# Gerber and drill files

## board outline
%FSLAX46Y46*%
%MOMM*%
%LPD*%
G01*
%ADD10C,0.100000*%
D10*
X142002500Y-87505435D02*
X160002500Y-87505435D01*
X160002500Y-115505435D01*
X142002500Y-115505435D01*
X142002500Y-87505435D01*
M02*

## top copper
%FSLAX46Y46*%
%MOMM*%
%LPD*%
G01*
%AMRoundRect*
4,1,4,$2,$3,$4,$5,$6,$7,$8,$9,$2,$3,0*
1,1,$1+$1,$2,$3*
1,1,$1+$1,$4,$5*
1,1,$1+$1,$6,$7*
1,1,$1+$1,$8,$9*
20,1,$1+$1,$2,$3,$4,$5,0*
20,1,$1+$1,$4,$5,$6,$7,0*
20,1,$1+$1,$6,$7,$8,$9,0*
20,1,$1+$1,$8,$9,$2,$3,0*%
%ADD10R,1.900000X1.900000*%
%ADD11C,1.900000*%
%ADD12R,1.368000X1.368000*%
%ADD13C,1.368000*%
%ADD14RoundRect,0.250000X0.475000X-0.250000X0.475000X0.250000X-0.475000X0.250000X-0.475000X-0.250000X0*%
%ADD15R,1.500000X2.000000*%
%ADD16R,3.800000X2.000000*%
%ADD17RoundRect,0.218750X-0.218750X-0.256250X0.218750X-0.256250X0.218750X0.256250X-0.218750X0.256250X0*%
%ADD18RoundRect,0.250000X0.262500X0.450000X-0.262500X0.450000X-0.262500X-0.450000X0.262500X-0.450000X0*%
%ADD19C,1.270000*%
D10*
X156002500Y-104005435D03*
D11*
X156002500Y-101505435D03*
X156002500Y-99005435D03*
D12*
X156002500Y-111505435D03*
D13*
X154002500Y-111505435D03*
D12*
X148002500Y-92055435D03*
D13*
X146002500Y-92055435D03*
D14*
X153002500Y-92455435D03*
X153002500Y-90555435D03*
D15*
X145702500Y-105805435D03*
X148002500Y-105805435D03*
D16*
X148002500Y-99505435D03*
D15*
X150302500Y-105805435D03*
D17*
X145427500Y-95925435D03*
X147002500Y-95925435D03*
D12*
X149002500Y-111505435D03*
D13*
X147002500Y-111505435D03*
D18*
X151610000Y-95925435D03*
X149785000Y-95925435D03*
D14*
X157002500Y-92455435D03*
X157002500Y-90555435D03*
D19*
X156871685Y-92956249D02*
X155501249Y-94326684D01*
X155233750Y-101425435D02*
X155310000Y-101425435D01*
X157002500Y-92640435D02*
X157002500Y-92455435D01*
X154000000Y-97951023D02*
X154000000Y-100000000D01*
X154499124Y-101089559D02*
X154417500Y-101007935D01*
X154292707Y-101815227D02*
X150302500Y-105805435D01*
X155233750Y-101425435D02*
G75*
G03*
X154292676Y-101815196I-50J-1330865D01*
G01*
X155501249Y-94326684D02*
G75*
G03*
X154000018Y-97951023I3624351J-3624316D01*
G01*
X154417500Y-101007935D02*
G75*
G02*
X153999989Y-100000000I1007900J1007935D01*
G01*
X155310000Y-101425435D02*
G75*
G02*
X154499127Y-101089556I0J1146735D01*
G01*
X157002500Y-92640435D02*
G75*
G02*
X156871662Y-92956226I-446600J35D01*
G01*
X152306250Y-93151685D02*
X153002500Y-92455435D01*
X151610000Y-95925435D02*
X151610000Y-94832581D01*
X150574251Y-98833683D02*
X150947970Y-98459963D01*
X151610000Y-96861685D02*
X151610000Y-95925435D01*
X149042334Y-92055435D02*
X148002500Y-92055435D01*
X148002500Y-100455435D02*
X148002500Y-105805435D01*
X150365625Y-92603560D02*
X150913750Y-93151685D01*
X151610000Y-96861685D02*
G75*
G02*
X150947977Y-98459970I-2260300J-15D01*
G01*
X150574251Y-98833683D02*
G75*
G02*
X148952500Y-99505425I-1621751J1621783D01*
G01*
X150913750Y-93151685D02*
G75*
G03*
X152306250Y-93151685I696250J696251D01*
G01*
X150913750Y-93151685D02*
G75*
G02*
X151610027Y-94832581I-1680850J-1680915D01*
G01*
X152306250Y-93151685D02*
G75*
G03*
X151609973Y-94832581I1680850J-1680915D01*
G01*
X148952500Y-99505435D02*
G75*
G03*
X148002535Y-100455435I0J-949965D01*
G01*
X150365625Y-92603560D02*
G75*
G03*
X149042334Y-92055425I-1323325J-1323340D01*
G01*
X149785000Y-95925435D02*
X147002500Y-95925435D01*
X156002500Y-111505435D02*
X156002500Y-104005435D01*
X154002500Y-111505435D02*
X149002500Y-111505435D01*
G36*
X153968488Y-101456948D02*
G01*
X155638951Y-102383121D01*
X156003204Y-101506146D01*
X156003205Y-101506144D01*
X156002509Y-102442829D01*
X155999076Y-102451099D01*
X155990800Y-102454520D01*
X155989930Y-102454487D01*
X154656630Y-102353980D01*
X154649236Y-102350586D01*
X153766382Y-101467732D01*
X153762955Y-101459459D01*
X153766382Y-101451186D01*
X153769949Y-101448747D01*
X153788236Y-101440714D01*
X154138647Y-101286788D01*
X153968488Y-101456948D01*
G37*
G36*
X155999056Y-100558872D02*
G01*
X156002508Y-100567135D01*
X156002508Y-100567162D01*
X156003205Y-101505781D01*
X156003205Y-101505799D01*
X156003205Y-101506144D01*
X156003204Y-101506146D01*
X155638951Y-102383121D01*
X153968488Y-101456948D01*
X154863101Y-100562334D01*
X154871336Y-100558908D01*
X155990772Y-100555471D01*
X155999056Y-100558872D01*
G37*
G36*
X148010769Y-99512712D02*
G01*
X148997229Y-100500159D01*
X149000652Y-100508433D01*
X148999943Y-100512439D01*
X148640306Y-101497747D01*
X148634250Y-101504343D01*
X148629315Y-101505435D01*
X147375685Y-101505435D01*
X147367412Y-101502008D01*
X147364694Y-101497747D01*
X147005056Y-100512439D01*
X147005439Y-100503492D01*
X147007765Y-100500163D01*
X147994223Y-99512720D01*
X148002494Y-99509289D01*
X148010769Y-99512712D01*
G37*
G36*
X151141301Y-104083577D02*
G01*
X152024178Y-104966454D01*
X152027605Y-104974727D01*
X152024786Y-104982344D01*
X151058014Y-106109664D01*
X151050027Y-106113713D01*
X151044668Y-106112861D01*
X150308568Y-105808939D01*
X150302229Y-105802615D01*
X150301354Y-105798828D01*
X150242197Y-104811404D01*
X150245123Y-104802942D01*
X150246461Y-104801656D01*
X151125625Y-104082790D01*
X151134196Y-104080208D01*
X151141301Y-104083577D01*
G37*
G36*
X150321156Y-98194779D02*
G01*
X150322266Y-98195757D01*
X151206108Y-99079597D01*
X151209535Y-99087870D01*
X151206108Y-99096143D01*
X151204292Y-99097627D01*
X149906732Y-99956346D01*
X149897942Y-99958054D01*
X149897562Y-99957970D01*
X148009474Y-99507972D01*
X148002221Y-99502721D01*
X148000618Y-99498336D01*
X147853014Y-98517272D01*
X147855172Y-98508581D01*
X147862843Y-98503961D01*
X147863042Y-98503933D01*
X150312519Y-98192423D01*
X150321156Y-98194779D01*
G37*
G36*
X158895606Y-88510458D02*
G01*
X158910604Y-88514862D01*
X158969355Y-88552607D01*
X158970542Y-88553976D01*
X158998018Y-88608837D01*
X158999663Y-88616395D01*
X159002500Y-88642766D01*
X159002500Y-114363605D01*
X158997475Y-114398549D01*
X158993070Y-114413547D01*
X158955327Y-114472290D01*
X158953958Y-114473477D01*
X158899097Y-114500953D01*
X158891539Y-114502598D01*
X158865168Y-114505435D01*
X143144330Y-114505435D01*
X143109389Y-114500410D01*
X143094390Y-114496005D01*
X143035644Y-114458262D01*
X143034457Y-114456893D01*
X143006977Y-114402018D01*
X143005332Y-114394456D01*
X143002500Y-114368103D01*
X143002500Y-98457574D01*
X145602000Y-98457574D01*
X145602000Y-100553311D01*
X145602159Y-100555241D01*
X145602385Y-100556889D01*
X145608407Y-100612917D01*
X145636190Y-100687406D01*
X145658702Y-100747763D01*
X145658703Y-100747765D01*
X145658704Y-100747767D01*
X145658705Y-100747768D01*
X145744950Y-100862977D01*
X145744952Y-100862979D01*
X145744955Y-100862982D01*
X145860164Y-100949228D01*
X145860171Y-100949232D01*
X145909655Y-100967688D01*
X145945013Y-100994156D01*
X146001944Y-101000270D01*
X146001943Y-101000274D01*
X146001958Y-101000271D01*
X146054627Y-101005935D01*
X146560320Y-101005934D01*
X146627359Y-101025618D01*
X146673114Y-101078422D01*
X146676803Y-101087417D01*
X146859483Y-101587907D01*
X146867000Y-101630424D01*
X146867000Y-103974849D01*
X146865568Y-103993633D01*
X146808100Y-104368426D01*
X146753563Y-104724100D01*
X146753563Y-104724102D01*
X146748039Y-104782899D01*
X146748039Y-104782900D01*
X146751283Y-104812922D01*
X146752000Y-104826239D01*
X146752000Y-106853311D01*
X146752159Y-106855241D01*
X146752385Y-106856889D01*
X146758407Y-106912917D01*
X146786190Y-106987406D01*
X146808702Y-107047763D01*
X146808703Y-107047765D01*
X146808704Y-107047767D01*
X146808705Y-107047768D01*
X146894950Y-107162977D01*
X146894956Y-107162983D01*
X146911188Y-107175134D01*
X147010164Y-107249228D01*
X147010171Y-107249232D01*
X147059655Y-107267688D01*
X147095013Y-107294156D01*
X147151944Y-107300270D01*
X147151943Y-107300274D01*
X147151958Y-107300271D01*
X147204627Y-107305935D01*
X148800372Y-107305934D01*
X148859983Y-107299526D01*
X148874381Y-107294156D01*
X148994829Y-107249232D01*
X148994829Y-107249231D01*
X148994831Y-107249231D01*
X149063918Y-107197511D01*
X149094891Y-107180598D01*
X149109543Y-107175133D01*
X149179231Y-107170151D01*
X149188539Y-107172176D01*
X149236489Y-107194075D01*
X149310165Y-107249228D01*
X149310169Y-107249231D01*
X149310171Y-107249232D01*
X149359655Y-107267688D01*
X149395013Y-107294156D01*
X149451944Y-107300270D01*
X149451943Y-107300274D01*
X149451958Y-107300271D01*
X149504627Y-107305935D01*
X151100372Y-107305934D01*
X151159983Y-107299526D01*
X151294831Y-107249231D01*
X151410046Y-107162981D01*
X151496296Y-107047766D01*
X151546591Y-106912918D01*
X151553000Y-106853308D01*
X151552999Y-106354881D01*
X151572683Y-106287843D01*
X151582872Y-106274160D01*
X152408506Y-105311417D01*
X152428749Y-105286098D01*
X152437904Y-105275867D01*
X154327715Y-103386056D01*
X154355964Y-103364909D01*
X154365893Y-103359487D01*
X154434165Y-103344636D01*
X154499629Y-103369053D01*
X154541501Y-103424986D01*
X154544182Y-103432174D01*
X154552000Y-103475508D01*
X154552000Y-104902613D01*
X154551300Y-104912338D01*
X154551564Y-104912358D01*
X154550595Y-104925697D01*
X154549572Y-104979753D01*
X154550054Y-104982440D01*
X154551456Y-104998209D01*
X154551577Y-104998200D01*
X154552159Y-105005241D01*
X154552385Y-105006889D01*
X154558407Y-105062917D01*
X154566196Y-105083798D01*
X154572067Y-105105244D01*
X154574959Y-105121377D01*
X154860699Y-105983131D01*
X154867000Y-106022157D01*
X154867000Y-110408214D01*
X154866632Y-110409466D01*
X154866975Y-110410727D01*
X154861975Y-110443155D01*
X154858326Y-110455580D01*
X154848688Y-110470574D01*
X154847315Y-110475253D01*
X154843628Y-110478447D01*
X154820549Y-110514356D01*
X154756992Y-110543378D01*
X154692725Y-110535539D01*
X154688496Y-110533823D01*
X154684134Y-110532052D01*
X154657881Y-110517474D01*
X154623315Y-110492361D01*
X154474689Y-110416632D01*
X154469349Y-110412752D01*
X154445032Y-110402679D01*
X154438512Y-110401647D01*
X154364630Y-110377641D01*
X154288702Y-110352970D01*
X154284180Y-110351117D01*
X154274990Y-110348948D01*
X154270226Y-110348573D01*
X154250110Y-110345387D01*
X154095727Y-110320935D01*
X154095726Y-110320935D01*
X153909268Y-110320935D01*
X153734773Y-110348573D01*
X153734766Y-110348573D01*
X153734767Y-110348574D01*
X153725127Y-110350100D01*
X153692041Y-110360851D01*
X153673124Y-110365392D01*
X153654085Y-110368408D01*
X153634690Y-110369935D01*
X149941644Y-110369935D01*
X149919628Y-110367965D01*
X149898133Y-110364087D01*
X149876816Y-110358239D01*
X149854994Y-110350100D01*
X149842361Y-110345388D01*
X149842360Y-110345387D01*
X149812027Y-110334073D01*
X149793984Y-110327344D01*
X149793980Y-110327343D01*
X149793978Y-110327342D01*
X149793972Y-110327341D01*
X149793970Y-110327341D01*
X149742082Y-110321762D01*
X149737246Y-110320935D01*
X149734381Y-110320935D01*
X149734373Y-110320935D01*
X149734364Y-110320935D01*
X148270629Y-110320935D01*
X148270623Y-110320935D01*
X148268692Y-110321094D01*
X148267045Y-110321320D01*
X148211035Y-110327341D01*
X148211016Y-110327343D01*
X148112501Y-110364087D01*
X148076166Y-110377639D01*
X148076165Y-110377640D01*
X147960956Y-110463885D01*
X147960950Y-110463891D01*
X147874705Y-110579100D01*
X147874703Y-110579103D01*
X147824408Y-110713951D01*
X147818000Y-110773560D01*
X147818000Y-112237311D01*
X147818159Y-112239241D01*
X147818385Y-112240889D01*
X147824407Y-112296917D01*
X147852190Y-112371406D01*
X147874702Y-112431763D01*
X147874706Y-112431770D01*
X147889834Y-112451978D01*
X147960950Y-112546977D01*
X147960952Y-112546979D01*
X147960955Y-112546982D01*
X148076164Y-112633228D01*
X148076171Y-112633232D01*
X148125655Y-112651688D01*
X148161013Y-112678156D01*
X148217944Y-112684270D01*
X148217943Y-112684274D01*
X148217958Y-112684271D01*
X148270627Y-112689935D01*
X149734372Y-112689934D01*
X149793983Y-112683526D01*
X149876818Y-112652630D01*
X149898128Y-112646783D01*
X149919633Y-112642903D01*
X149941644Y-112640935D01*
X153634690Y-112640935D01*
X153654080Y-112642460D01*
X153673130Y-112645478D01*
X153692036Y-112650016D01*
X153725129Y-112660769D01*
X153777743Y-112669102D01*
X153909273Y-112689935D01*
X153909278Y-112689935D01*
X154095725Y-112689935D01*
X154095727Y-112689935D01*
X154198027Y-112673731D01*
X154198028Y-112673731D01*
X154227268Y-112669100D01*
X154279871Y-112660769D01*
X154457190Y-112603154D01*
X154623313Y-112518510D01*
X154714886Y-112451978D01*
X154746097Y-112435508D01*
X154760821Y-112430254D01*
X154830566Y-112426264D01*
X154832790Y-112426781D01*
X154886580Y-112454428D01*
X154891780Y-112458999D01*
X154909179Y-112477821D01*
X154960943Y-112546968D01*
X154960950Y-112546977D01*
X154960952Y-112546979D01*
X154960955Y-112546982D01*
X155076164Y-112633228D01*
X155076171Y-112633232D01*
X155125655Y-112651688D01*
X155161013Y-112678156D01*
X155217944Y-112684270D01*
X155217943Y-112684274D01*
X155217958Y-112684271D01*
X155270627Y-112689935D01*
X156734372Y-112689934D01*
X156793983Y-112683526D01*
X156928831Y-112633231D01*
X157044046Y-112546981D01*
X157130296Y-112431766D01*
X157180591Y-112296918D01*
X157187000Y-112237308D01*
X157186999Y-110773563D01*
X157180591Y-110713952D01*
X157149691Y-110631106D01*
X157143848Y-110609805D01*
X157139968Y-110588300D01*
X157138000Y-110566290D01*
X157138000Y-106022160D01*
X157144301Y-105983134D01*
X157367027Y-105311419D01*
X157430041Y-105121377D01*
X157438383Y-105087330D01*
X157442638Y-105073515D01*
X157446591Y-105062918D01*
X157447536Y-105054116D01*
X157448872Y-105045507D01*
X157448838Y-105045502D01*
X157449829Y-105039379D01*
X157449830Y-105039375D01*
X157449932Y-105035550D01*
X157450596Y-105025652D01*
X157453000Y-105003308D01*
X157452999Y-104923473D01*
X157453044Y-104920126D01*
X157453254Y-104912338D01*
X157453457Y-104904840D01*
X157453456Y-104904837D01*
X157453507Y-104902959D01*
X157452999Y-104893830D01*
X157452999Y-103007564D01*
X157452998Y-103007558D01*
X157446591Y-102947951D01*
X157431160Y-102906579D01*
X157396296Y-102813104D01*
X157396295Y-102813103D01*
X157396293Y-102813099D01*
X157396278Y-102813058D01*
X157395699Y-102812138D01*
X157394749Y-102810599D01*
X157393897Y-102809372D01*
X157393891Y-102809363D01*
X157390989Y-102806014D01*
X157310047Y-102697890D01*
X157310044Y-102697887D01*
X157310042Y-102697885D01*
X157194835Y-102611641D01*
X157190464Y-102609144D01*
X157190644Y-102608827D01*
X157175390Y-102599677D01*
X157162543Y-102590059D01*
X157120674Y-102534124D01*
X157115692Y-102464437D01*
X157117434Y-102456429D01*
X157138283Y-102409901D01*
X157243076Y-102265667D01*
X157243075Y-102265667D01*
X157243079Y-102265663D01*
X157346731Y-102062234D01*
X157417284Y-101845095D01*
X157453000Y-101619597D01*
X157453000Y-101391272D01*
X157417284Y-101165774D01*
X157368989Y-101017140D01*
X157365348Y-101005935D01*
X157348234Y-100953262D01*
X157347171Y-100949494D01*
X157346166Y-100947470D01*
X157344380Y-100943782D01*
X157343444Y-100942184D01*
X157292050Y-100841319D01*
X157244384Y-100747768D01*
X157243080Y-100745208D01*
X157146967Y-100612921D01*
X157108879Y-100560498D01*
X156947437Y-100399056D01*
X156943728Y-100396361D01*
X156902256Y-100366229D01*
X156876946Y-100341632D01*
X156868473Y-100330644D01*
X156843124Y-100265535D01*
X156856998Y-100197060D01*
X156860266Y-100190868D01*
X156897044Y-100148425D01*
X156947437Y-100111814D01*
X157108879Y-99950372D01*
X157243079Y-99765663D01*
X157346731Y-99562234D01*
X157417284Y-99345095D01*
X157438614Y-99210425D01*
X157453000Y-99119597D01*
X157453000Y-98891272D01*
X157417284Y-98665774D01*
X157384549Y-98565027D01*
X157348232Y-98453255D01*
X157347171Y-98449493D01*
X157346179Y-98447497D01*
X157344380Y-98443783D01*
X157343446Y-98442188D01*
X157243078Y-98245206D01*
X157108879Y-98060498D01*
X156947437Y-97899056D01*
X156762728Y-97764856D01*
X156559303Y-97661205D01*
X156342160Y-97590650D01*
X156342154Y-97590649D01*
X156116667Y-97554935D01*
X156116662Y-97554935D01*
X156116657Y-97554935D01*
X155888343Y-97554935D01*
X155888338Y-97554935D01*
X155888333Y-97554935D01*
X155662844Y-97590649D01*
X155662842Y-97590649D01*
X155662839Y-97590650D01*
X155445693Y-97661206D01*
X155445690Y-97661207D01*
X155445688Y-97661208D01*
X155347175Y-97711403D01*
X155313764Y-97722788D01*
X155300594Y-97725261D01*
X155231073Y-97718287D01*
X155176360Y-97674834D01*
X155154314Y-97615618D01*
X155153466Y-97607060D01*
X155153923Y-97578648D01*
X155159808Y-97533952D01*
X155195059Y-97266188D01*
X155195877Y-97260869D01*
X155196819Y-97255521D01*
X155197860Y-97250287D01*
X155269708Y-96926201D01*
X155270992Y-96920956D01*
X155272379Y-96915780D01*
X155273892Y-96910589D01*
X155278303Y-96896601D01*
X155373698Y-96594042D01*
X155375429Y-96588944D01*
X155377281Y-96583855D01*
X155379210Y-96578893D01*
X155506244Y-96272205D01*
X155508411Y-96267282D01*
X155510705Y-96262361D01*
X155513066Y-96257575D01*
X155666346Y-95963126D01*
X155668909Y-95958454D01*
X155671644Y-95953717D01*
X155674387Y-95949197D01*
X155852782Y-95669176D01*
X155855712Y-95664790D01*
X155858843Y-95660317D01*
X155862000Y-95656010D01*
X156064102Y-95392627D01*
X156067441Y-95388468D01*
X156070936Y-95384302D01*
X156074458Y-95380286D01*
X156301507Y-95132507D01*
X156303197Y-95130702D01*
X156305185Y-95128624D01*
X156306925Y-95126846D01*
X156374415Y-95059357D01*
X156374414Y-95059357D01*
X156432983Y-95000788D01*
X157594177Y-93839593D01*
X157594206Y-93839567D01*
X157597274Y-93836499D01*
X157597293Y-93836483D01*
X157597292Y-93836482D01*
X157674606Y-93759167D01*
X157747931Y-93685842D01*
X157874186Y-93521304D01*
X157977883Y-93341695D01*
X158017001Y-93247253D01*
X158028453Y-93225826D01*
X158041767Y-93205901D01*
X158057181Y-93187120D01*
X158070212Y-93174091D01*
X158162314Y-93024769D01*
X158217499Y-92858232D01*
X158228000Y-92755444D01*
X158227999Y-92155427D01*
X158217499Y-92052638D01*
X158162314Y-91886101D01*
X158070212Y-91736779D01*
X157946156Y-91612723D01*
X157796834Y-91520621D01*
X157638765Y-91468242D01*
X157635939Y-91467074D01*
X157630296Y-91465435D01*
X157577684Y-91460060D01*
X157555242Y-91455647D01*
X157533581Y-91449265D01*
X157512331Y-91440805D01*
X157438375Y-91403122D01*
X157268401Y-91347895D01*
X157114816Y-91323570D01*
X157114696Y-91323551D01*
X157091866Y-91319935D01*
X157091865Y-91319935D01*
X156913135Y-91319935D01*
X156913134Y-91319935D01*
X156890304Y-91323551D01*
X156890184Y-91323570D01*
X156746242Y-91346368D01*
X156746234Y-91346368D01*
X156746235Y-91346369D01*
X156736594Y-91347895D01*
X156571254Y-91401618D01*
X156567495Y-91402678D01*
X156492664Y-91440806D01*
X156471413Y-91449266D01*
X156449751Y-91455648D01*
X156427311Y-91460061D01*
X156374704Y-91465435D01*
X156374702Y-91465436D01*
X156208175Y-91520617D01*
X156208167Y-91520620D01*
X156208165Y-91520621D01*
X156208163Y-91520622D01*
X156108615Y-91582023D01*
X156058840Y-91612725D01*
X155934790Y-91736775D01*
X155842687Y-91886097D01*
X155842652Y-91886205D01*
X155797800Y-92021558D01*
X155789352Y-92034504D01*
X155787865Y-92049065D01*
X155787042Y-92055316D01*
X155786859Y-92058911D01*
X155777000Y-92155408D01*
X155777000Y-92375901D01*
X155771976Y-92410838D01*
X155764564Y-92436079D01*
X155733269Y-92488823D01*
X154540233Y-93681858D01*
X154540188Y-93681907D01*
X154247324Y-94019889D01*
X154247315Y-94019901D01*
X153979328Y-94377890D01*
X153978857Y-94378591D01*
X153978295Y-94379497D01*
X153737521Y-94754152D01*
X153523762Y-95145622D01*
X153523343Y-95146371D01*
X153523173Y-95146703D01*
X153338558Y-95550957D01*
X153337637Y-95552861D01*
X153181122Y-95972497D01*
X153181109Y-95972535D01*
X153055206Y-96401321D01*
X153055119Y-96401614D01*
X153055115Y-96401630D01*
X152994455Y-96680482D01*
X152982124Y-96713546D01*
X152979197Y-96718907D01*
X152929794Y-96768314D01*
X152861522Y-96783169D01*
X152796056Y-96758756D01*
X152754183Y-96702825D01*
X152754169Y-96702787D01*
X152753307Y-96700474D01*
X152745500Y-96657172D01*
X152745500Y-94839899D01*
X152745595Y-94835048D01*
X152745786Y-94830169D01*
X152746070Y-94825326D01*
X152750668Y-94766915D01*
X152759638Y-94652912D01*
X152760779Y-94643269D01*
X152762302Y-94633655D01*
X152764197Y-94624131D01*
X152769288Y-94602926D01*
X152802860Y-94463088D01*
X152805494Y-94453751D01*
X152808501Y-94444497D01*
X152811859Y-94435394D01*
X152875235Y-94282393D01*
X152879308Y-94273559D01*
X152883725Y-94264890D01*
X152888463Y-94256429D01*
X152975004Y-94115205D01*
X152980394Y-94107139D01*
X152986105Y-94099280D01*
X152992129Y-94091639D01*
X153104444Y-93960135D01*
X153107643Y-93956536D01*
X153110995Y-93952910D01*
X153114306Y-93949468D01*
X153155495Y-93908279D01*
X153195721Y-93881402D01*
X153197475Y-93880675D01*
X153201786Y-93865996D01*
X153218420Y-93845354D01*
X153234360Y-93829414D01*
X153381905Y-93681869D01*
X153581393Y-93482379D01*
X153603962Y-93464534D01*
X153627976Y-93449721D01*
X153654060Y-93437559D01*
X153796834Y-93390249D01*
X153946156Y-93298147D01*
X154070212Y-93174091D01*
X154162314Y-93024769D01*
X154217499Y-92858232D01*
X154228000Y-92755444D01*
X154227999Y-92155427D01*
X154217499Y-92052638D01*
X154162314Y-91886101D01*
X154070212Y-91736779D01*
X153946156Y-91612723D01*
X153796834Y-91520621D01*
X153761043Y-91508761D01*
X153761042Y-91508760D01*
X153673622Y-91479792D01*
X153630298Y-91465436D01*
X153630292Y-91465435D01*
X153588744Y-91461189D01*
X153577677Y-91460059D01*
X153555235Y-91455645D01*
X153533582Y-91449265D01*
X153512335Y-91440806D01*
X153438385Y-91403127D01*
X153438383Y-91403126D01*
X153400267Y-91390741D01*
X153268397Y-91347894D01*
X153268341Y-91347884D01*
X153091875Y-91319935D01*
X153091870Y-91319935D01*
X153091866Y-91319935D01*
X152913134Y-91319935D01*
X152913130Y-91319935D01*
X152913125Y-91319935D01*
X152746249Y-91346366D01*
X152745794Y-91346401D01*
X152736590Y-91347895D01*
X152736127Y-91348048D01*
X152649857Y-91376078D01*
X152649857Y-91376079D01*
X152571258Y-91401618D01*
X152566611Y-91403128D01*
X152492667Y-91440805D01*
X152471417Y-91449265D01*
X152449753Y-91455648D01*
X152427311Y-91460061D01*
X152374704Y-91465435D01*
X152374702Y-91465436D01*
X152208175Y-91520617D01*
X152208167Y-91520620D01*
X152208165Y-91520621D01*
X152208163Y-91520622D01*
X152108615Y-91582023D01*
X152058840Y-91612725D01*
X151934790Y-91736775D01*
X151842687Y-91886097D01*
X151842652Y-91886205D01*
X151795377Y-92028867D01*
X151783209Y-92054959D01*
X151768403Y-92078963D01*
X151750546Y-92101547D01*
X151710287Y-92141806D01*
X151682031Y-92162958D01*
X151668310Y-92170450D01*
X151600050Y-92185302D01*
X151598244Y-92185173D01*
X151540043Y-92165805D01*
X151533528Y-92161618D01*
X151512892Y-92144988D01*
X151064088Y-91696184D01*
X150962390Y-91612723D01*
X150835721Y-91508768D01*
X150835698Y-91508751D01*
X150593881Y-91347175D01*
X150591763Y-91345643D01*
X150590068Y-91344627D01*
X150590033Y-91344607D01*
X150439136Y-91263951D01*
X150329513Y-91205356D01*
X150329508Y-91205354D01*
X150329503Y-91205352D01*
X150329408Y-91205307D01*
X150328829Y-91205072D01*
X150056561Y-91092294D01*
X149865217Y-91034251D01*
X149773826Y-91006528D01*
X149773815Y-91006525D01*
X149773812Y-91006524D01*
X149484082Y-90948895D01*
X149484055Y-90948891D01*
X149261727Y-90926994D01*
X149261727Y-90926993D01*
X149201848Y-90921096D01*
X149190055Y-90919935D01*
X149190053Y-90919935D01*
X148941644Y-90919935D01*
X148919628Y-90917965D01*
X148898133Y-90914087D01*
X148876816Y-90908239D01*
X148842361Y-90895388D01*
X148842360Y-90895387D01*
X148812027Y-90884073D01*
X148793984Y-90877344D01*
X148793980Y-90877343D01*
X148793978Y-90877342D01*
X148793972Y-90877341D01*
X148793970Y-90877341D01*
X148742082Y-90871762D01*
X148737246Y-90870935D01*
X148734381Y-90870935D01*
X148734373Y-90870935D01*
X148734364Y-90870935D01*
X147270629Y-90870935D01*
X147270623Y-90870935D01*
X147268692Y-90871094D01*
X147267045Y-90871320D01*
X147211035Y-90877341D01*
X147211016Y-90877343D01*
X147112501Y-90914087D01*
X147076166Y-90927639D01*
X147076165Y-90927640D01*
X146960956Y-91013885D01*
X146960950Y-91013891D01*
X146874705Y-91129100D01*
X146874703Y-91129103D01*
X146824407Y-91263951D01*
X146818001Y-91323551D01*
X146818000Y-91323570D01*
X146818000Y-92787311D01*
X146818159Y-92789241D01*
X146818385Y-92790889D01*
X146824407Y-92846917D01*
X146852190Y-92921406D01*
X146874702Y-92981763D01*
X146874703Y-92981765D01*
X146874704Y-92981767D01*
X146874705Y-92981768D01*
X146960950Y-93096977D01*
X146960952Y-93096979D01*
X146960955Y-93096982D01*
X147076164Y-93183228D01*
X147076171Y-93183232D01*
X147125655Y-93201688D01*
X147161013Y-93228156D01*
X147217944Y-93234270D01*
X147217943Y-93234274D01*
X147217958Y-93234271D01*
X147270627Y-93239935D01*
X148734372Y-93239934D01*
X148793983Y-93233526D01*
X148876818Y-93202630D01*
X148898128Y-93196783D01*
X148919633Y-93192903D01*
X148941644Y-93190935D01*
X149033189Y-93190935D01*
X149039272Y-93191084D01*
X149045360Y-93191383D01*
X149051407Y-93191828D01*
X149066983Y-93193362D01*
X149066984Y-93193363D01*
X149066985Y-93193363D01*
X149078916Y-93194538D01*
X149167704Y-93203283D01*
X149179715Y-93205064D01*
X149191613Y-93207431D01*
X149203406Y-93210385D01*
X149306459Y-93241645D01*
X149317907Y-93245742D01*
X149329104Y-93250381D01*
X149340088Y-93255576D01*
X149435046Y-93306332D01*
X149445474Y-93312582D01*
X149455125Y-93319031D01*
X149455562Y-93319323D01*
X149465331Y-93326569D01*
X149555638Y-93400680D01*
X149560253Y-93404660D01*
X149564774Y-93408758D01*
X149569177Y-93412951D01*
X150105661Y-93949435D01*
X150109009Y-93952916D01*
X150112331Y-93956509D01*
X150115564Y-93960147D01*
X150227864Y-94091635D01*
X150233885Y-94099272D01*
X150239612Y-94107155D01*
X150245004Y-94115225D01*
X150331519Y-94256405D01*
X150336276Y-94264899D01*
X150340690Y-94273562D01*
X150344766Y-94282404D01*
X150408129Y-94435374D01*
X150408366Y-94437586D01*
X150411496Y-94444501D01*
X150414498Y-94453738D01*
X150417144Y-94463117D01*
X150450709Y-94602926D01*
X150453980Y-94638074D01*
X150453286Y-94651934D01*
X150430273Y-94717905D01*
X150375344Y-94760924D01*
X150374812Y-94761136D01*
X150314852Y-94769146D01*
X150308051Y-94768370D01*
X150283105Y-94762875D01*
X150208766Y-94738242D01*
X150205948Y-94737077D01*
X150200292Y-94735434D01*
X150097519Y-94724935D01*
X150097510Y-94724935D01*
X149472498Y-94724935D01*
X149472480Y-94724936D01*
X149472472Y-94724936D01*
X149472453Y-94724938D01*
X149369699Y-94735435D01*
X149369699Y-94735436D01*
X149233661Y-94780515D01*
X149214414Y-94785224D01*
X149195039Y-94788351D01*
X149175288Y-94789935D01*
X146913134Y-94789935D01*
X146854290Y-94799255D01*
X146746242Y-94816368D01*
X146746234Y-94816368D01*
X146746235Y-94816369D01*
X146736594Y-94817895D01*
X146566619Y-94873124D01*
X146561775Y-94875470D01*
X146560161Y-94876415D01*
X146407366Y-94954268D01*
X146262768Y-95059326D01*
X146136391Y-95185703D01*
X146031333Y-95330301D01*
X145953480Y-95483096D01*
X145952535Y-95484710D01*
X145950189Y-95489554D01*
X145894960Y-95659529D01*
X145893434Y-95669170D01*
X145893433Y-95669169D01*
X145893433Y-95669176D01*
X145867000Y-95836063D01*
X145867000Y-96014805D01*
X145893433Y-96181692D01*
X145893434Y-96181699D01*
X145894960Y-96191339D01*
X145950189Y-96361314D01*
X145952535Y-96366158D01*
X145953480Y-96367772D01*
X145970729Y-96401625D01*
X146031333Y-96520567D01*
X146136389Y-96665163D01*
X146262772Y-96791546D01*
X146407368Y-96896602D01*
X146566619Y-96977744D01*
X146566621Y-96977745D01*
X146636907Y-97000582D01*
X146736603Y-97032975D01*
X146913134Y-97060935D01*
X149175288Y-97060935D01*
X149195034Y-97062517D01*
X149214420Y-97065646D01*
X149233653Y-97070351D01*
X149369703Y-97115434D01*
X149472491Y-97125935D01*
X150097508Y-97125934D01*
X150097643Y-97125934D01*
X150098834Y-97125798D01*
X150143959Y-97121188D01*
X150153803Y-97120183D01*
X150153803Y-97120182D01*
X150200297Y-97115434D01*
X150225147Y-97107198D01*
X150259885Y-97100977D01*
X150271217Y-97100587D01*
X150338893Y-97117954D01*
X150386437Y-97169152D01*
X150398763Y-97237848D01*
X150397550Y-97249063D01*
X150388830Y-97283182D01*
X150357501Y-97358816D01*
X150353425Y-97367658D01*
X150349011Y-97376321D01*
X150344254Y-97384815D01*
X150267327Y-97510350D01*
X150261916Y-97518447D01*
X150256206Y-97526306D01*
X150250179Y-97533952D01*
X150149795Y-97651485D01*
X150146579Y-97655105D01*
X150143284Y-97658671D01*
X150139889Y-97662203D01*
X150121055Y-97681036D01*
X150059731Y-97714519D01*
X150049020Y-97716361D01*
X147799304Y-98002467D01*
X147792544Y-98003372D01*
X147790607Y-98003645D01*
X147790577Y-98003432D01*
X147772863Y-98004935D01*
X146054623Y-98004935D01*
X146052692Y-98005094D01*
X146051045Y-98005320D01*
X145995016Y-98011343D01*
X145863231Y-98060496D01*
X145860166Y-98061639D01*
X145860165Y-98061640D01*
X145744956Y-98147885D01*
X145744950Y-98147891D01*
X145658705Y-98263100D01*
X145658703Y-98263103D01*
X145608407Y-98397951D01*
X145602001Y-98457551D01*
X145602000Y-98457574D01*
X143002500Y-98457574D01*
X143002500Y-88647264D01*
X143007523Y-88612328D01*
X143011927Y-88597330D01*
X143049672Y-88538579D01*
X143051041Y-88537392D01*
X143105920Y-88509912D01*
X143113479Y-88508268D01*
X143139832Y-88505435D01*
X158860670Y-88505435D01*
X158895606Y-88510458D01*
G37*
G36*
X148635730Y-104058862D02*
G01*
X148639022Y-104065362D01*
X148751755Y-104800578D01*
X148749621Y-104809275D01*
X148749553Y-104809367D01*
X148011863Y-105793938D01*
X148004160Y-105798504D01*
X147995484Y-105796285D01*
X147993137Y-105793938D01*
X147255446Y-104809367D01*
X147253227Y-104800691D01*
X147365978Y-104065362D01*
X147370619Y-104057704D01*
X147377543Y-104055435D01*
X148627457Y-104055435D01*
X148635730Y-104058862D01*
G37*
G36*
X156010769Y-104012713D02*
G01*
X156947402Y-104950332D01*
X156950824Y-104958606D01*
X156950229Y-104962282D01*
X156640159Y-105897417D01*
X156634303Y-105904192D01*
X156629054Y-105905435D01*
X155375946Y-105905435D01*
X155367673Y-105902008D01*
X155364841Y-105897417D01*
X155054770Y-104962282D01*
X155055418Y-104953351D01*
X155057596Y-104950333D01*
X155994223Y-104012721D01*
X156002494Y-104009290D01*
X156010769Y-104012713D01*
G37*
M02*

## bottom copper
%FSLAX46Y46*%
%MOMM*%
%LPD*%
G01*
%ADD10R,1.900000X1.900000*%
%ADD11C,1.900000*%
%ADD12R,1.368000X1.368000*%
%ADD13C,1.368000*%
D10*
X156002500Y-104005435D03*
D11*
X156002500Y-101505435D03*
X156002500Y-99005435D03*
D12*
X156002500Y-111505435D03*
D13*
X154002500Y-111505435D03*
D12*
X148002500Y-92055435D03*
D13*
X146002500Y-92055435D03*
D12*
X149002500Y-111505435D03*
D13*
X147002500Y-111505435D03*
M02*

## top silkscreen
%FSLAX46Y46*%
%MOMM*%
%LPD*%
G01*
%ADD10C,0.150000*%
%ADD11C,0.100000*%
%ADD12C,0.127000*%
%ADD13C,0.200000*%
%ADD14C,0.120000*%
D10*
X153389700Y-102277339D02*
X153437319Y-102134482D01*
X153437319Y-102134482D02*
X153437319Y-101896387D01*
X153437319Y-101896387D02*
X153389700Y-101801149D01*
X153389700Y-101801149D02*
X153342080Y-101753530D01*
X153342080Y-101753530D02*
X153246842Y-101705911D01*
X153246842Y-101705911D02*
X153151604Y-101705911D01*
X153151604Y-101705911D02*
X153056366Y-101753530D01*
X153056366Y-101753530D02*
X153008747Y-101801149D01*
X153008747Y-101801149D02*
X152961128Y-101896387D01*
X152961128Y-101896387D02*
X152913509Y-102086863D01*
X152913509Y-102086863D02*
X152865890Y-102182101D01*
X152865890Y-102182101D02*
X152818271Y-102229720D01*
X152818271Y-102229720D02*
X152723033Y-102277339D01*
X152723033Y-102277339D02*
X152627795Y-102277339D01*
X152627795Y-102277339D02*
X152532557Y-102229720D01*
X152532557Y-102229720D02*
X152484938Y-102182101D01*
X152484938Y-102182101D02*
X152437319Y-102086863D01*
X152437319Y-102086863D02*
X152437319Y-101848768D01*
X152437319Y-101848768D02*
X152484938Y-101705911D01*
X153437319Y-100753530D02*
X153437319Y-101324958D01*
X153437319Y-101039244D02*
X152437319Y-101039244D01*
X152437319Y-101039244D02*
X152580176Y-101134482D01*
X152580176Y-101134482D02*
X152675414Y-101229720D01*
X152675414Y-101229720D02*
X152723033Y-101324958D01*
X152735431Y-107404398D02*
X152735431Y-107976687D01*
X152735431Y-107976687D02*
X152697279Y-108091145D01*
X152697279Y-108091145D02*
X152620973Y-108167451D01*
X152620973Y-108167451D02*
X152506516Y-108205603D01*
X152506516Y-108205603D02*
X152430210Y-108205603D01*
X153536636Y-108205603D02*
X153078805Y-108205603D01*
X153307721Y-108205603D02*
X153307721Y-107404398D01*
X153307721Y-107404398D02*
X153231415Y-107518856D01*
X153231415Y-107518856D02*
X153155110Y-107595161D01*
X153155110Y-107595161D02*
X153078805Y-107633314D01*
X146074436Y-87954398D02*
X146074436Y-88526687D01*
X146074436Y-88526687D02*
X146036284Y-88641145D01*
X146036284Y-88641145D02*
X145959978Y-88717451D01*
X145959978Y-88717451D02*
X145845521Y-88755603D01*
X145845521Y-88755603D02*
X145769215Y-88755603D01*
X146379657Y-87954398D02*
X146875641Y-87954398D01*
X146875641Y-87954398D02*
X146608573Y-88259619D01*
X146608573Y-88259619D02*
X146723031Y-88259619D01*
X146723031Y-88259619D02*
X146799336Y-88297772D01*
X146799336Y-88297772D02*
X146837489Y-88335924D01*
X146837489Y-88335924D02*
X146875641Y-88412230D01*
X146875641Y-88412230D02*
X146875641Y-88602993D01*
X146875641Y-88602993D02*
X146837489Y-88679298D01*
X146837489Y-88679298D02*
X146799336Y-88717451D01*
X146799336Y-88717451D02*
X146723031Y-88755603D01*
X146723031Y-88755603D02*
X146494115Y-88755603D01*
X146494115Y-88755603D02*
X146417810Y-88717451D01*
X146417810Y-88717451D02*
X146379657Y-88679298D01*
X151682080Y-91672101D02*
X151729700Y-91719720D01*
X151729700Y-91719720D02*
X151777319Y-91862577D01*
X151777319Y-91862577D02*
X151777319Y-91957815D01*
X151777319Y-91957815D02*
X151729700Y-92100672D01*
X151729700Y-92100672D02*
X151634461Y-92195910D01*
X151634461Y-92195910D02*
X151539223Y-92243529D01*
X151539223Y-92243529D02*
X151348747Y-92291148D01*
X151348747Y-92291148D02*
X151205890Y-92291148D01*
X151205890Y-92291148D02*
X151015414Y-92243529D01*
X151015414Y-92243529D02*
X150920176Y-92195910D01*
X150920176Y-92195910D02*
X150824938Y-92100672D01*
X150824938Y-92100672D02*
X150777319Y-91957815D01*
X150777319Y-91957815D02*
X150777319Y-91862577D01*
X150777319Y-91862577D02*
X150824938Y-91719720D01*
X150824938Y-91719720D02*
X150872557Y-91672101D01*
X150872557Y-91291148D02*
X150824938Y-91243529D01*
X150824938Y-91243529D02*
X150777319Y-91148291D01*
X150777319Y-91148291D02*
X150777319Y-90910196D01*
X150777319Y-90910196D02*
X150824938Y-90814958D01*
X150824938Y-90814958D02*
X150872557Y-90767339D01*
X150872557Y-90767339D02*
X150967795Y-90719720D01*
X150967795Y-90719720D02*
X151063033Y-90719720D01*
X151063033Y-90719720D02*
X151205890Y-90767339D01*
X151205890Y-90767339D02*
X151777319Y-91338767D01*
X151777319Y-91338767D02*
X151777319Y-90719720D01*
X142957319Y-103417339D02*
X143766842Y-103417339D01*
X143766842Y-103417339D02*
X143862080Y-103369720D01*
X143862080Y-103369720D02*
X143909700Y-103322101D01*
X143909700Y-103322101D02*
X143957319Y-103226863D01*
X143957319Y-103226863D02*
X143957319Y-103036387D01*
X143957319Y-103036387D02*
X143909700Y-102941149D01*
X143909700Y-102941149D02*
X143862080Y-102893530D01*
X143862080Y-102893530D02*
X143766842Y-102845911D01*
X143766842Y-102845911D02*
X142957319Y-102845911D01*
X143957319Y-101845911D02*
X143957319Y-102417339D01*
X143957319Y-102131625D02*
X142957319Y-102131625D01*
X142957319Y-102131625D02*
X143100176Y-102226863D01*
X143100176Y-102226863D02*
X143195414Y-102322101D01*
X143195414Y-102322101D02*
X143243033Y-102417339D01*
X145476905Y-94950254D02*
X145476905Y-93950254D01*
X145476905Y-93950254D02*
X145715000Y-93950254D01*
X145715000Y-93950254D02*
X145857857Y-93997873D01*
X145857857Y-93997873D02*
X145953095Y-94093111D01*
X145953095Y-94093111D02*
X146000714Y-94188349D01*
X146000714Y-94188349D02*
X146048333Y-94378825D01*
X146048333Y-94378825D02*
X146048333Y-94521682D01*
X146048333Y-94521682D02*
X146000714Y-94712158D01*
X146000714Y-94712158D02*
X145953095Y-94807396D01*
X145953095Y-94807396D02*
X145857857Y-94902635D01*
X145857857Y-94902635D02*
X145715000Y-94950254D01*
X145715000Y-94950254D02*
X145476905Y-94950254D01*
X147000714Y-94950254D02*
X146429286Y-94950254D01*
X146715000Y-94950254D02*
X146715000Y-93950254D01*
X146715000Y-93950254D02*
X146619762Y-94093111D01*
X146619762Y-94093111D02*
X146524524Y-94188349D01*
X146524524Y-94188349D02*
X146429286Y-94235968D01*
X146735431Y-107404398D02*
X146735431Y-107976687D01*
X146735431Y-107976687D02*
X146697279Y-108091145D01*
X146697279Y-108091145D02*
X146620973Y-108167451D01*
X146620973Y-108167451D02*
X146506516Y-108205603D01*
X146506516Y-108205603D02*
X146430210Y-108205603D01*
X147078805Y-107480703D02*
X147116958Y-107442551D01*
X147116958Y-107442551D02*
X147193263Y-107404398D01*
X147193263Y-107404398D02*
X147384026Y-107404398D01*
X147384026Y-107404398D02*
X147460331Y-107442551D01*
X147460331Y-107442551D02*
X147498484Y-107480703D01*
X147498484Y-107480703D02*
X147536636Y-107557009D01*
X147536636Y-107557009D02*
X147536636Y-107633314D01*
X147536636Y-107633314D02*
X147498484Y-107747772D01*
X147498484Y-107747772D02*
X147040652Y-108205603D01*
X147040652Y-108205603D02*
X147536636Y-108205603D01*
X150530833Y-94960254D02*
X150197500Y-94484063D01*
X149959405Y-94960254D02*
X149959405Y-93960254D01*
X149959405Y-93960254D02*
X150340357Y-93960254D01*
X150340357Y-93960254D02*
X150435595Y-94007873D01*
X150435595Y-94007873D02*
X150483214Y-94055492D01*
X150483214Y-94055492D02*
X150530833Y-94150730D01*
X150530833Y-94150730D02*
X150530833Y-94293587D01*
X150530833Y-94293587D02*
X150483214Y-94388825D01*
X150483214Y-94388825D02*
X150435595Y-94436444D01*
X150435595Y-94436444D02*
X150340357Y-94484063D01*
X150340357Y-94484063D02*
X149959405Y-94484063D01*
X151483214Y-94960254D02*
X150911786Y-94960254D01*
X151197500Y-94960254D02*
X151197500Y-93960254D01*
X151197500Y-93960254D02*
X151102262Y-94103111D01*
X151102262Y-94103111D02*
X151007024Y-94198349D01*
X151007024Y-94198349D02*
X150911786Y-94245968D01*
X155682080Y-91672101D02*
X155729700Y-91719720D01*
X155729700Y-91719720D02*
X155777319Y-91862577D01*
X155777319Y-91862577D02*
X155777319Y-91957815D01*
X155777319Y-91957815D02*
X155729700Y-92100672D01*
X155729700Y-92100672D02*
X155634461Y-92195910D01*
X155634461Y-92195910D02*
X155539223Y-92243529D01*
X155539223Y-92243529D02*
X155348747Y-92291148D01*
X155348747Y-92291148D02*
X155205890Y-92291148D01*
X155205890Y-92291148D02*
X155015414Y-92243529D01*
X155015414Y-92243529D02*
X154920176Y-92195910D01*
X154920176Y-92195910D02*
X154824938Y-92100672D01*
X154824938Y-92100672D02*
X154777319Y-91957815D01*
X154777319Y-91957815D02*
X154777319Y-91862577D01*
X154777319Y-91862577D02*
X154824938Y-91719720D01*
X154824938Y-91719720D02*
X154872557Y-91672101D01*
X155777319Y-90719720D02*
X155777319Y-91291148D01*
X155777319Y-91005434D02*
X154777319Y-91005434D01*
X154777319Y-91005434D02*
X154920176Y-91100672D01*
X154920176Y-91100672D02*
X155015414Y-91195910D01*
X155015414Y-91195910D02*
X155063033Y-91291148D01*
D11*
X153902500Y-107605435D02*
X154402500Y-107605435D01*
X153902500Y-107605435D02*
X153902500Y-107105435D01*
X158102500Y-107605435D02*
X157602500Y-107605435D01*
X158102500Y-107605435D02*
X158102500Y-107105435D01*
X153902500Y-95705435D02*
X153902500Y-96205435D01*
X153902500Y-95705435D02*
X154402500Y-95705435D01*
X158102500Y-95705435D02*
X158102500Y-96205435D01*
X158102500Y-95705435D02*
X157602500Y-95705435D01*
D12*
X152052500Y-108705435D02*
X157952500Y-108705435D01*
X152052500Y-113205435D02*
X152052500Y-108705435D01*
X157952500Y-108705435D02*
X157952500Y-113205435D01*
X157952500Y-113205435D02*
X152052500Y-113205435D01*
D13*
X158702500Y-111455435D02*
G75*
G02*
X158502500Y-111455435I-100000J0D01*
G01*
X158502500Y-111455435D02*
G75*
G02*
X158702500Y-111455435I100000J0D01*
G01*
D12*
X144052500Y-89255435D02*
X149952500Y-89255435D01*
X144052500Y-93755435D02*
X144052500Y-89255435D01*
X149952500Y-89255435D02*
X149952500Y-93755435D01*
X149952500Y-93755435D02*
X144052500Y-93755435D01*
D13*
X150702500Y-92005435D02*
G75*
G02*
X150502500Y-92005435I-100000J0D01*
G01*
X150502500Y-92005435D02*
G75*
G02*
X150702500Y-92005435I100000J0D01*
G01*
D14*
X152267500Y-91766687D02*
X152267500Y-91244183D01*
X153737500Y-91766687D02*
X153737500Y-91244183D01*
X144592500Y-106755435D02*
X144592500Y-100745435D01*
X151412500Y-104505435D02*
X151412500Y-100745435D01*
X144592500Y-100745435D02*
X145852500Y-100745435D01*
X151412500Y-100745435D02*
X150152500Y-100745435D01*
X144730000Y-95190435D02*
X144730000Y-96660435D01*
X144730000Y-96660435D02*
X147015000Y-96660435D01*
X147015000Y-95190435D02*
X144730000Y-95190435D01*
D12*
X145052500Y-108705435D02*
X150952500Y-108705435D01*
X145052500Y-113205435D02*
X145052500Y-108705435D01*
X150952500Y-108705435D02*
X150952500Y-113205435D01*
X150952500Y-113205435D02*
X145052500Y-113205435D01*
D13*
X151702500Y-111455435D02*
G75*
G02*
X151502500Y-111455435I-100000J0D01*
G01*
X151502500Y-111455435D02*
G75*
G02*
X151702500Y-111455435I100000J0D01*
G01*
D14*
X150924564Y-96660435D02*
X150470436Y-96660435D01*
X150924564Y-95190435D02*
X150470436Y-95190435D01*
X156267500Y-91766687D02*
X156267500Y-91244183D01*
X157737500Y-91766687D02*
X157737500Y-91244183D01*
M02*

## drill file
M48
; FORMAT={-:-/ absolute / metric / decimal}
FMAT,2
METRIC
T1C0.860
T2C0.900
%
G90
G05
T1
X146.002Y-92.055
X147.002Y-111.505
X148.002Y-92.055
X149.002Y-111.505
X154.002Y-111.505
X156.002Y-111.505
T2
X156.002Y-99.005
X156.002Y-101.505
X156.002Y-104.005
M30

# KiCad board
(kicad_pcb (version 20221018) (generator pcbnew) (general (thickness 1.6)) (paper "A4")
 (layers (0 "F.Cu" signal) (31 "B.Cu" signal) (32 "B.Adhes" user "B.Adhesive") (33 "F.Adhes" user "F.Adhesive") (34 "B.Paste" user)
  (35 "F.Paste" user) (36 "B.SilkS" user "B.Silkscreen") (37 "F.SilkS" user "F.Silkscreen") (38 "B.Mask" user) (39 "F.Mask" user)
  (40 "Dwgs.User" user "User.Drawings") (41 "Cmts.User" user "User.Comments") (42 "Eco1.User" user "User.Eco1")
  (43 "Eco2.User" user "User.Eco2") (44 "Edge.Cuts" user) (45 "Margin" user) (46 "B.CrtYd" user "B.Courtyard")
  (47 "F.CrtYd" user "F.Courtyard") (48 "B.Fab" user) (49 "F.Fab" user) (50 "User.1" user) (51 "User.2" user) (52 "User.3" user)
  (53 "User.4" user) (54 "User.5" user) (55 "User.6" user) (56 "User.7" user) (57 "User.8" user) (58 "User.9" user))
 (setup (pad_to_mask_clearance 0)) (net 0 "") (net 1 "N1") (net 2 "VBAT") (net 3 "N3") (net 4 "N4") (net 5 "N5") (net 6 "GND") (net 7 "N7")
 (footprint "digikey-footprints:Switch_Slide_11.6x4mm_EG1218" (layer "F.Cu") (at 156.0025 104.005435 90)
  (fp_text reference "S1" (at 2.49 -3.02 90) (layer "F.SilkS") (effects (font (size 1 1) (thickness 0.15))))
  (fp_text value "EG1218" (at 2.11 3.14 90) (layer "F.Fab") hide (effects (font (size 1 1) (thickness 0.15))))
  (fp_line (start -3.6 -2.1) (end -3.6 -1.6) (stroke (width 0.1) (type solid)) (layer "F.SilkS"))
  (fp_line (start -3.6 -2.1) (end -3.1 -2.1) (stroke (width 0.1) (type solid)) (layer "F.SilkS"))
  (fp_line (start -3.6 2.1) (end -3.6 1.6) (stroke (width 0.1) (type solid)) (layer "F.SilkS"))
  (fp_line (start -3.6 2.1) (end -3.1 2.1) (stroke (width 0.1) (type solid)) (layer "F.SilkS"))
  (fp_line (start 8.3 -2.1) (end 7.8 -2.1) (stroke (width 0.1) (type solid)) (layer "F.SilkS"))
  (fp_line (start 8.3 -2.1) (end 8.3 -1.6) (stroke (width 0.1) (type solid)) (layer "F.SilkS"))
  (fp_line (start 8.3 2.1) (end 7.8 2.1) (stroke (width 0.1) (type solid)) (layer "F.SilkS"))
  (fp_line (start 8.3 2.1) (end 8.3 1.6) (stroke (width 0.1) (type solid)) (layer "F.SilkS"))
  (pad "1" thru_hole rect (at 0 0 90) (size 1.9 1.9) (drill 0.9) (layers "*.Cu" "*.Mask") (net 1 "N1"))
  (pad "2" thru_hole circle (at 2.5 0 90) (size 1.9 1.9) (drill 0.9) (layers "*.Cu" "*.Mask") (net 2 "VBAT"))
  (pad "3" thru_hole circle (at 5 0 90) (size 1.9 1.9) (drill 0.9) (layers "*.Cu" "*.Mask") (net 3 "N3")))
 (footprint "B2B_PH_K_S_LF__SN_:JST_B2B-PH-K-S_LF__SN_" (layer "F.Cu") (at 155.0025 110.955435)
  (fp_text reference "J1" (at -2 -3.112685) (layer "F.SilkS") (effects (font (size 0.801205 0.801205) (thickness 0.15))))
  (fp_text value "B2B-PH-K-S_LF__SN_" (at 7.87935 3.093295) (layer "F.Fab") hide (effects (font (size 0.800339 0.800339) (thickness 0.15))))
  (fp_line (start -2.95 -2.25) (end 2.95 -2.25) (stroke (width 0.127) (type solid)) (layer "F.SilkS"))
  (fp_line (start -2.95 2.25) (end -2.95 -2.25) (stroke (width 0.127) (type solid)) (layer "F.SilkS"))
  (fp_line (start 2.95 -2.25) (end 2.95 2.25) (stroke (width 0.127) (type solid)) (layer "F.SilkS"))
  (fp_line (start 2.95 2.25) (end -2.95 2.25) (stroke (width 0.127) (type solid)) (layer "F.SilkS"))
  (fp_circle (center 3.6 0.5) (end 3.7 0.5) (stroke (width 0.2) (type solid)) (fill none) (layer "F.SilkS"))
  (pad "1" thru_hole rect (at 1 0.55) (size 1.368 1.368) (drill 0.86) (layers "*.Cu" "*.Mask") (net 1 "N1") (solder_mask_margin 0.102))
  (pad "2" thru_hole circle (at -1 0.55) (size 1.368 1.368) (drill 0.86) (layers "*.Cu" "*.Mask") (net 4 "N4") (solder_mask_margin 0.102)))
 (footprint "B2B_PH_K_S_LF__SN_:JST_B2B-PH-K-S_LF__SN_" (layer "F.Cu") (at 147.0025 91.505435)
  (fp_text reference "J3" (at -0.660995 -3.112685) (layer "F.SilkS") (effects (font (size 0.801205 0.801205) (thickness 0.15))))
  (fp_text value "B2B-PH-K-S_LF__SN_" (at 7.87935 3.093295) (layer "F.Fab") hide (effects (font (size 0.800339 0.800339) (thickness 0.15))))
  (fp_line (start -2.95 -2.25) (end 2.95 -2.25) (stroke (width 0.127) (type solid)) (layer "F.SilkS"))
  (fp_line (start -2.95 2.25) (end -2.95 -2.25) (stroke (width 0.127) (type solid)) (layer "F.SilkS"))
  (fp_line (start 2.95 -2.25) (end 2.95 2.25) (stroke (width 0.127) (type solid)) (layer "F.SilkS"))
  (fp_line (start 2.95 2.25) (end -2.95 2.25) (stroke (width 0.127) (type solid)) (layer "F.SilkS"))
  (fp_circle (center 3.6 0.5) (end 3.7 0.5) (stroke (width 0.2) (type solid)) (fill none) (layer "F.SilkS"))
  (pad "1" thru_hole rect (at 1 0.55) (size 1.368 1.368) (drill 0.86) (layers "*.Cu" "*.Mask") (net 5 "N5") (solder_mask_margin 0.102))
  (pad "2" thru_hole circle (at -1 0.55) (size 1.368 1.368) (drill 0.86) (layers "*.Cu" "*.Mask") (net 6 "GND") (solder_mask_margin 0.102)))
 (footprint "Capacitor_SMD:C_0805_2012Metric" (layer "F.Cu") (at 153.0025 91.505435 90)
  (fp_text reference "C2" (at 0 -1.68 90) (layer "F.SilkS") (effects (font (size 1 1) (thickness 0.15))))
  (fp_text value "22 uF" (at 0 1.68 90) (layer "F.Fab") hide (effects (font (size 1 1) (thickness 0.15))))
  (fp_line (start -0.261252 -0.735) (end 0.261252 -0.735) (stroke (width 0.12) (type solid)) (layer "F.SilkS"))
  (fp_line (start -0.261252 0.735) (end 0.261252 0.735) (stroke (width 0.12) (type solid)) (layer "F.SilkS"))
  (pad "1" smd roundrect (at -0.95 0 90) (size 1 1.45) (layers "F.Cu" "F.Paste" "F.Mask") (roundrect_rratio 0.25) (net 5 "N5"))
  (pad "2" smd roundrect (at 0.95 0 90) (size 1 1.45) (layers "F.Cu" "F.Paste" "F.Mask") (roundrect_rratio 0.25) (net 6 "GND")))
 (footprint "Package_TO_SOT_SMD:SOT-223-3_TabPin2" (layer "F.Cu") (at 148.0025 102.655435 90)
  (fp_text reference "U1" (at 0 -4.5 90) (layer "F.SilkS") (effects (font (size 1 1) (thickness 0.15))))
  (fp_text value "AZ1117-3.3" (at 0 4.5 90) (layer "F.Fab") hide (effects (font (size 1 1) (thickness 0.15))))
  (fp_line (start -4.1 -3.41) (end 1.91 -3.41) (stroke (width 0.12) (type solid)) (layer "F.SilkS"))
  (fp_line (start -1.85 3.41) (end 1.91 3.41) (stroke (width 0.12) (type solid)) (layer "F.SilkS"))
  (fp_line (start 1.91 -3.41) (end 1.91 -2.15) (stroke (width 0.12) (type solid)) (layer "F.SilkS"))
  (fp_line (start 1.91 3.41) (end 1.91 2.15) (stroke (width 0.12) (type solid)) (layer "F.SilkS"))
  (pad "1" smd rect (at -3.15 -2.3 90) (size 2 1.5) (layers "F.Cu" "F.Paste" "F.Mask") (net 6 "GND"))
  (pad "2" smd rect (at -3.15 0 90) (size 2 1.5) (layers "F.Cu" "F.Paste" "F.Mask") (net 5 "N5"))
  (pad "2" smd rect (at 3.15 0 90) (size 2 3.8) (layers "F.Cu" "F.Paste" "F.Mask") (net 5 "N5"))
  (pad "3" smd rect (at -3.15 2.3 90) (size 2 1.5) (layers "F.Cu" "F.Paste" "F.Mask") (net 2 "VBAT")))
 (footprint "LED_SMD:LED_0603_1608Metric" (layer "F.Cu") (at 146.215 95.925435)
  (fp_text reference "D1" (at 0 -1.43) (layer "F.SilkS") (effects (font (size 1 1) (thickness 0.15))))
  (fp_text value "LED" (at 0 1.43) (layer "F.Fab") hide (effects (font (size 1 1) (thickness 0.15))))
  (fp_line (start -1.485 -0.735) (end -1.485 0.735) (stroke (width 0.12) (type solid)) (layer "F.SilkS"))
  (fp_line (start -1.485 0.735) (end 0.8 0.735) (stroke (width 0.12) (type solid)) (layer "F.SilkS"))
  (fp_line (start 0.8 -0.735) (end -1.485 -0.735) (stroke (width 0.12) (type solid)) (layer "F.SilkS"))
  (pad "1" smd roundrect (at -0.7875 0) (size 0.875 0.95) (layers "F.Cu" "F.Paste" "F.Mask") (roundrect_rratio 0.25) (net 6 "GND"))
  (pad "2" smd roundrect (at 0.7875 0) (size 0.875 0.95) (layers "F.Cu" "F.Paste" "F.Mask") (roundrect_rratio 0.25) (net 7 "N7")))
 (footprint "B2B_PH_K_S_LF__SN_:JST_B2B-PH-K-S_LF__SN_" (layer "F.Cu") (at 148.0025 110.955435)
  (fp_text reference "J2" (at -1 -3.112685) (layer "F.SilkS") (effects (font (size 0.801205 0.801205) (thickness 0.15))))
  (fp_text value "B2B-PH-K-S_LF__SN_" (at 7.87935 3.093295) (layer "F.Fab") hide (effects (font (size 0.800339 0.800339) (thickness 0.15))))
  (fp_line (start -2.95 -2.25) (end 2.95 -2.25) (stroke (width 0.127) (type solid)) (layer "F.SilkS"))
  (fp_line (start -2.95 2.25) (end -2.95 -2.25) (stroke (width 0.127) (type solid)) (layer "F.SilkS"))
  (fp_line (start 2.95 -2.25) (end 2.95 2.25) (stroke (width 0.127) (type solid)) (layer "F.SilkS"))
  (fp_line (start 2.95 2.25) (end -2.95 2.25) (stroke (width 0.127) (type solid)) (layer "F.SilkS"))
  (fp_circle (center 3.6 0.5) (end 3.7 0.5) (stroke (width 0.2) (type solid)) (fill none) (layer "F.SilkS"))
  (pad "1" thru_hole rect (at 1 0.55) (size 1.368 1.368) (drill 0.86) (layers "*.Cu" "*.Mask") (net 4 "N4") (solder_mask_margin 0.102))
  (pad "2" thru_hole circle (at -1 0.55) (size 1.368 1.368) (drill 0.86) (layers "*.Cu" "*.Mask") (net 6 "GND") (solder_mask_margin 0.102)))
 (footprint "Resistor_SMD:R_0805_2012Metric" (layer "F.Cu") (at 150.6975 95.925435 180)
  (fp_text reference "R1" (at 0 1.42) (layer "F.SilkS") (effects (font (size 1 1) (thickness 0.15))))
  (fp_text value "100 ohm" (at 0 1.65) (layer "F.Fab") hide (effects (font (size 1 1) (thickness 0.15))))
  (fp_line (start -0.227064 -0.735) (end 0.227064 -0.735) (stroke (width 0.12) (type solid)) (layer "F.SilkS"))
  (fp_line (start -0.227064 0.735) (end 0.227064 0.735) (stroke (width 0.12) (type solid)) (layer "F.SilkS"))
  (pad "1" smd roundrect (at -0.9125 0 180) (size 1.025 1.4) (layers "F.Cu" "F.Paste" "F.Mask") (roundrect_rratio 0.243902) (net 5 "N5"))
  (pad "2" smd roundrect (at 0.9125 0 180) (size 1.025 1.4) (layers "F.Cu" "F.Paste" "F.Mask") (roundrect_rratio 0.243902) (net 7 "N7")))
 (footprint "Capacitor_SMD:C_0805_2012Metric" (layer "F.Cu") (at 157.0025 91.505435 90)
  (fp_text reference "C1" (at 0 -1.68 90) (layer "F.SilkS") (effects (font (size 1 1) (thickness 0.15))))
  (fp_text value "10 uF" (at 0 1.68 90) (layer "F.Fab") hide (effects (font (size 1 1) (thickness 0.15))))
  (fp_line (start -0.261252 -0.735) (end 0.261252 -0.735) (stroke (width 0.12) (type solid)) (layer "F.SilkS"))
  (fp_line (start -0.261252 0.735) (end 0.261252 0.735) (stroke (width 0.12) (type solid)) (layer "F.SilkS"))
  (pad "1" smd roundrect (at -0.95 0 90) (size 1 1.45) (layers "F.Cu" "F.Paste" "F.Mask") (roundrect_rratio 0.25) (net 2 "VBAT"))
  (pad "2" smd roundrect (at 0.95 0 90) (size 1 1.45) (layers "F.Cu" "F.Paste" "F.Mask") (roundrect_rratio 0.25) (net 6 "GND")))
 (gr_rect (start 142.0025 87.505435) (end 160.0025 115.505435) (stroke (width 0.1) (type default)) (fill none) (layer "Edge.Cuts"))
 (segment (start 156.871685 92.956249) (end 155.501249 94.326684) (width 1.27) (layer "F.Cu") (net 2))
 (segment (start 155.23375 101.425435) (end 155.31 101.425435) (width 1.27) (layer "F.Cu") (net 2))
 (segment (start 157.0025 92.640435) (end 157.0025 92.455435) (width 1.27) (layer "F.Cu") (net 2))
 (segment (start 154 97.951023) (end 154 100) (width 1.27) (layer "F.Cu") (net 2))
 (segment (start 154.499124 101.089559) (end 154.4175 101.007935) (width 1.27) (layer "F.Cu") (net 2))
 (segment (start 154.292707 101.815227) (end 150.3025 105.805435) (width 1.27) (layer "F.Cu") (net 2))
 (arc (start 155.23375 101.425435) (mid 154.724461 101.526738) (end 154.292707 101.815227) (width 1.27) (layer "F.Cu") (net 2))
 (arc (start 155.501249 94.326684) (mid 154.390161 95.989545) (end 154 97.951023) (width 1.27) (layer "F.Cu") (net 2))
 (arc (start 154.4175 101.007935) (mid 154.108504 100.54549) (end 154 100) (width 1.27) (layer "F.Cu") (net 2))
 (arc (start 155.31 101.425435) (mid 154.871157 101.338143) (end 154.499124 101.089559) (width 1.27) (layer "F.Cu") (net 2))
 (arc (start 157.0025 92.640435) (mid 156.968502 92.811352) (end 156.871685 92.956249) (width 1.27) (layer "F.Cu") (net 2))
 (segment (start 152.30625 93.151685) (end 153.0025 92.455435) (width 1.27) (layer "F.Cu") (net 5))
 (segment (start 151.61 95.925435) (end 151.61 94.832581) (width 1.27) (layer "F.Cu") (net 5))
 (segment (start 150.574251 98.833683) (end 150.94797 98.459963) (width 1.27) (layer "F.Cu") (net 5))
 (segment (start 151.61 96.861685) (end 151.61 95.925435) (width 1.27) (layer "F.Cu") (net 5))
 (segment (start 149.042334 92.055435) (end 148.0025 92.055435) (width 1.27) (layer "F.Cu") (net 5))
 (segment (start 148.0025 100.455435) (end 148.0025 105.805435) (width 1.27) (layer "F.Cu") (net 5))
 (segment (start 150.365625 92.60356) (end 150.91375 93.151685) (width 1.27) (layer "F.Cu") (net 5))
 (arc (start 151.61 96.861685) (mid 151.437944 97.726667) (end 150.94797 98.459963) (width 1.27) (layer "F.Cu") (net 5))
 (arc (start 150.574251 98.833683) (mid 149.830185 99.330852) (end 148.9525 99.505435) (width 1.27) (layer "F.Cu") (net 5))
 (arc (start 150.91375 93.151685) (mid 151.61 93.440081) (end 152.30625 93.151685) (width 1.27) (layer "F.Cu") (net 5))
 (arc (start 150.91375 93.151685) (mid 151.42905 93.922886) (end 151.61 94.832581) (width 1.27) (layer "F.Cu") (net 5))
 (arc (start 152.30625 93.151685) (mid 151.790949 93.922886) (end 151.61 94.832581) (width 1.27) (layer "F.Cu") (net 5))
 (arc (start 148.9525 99.505435) (mid 148.280748 99.783683) (end 148.0025 100.455435) (width 1.27) (layer "F.Cu") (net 5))
 (arc (start 150.365625 92.60356) (mid 149.758493 92.197888) (end 149.042334 92.055435) (width 1.27) (layer "F.Cu") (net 5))
 (segment (start 149.785 95.925435) (end 147.0025 95.925435) (width 1.27) (layer "F.Cu") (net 7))
 (segment (start 156.0025 111.505435) (end 156.0025 104.005435) (width 1.27) (layer "F.Cu") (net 1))
 (segment (start 154.0025 111.505435) (end 149.0025 111.505435) (width 1.27) (layer "F.Cu") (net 4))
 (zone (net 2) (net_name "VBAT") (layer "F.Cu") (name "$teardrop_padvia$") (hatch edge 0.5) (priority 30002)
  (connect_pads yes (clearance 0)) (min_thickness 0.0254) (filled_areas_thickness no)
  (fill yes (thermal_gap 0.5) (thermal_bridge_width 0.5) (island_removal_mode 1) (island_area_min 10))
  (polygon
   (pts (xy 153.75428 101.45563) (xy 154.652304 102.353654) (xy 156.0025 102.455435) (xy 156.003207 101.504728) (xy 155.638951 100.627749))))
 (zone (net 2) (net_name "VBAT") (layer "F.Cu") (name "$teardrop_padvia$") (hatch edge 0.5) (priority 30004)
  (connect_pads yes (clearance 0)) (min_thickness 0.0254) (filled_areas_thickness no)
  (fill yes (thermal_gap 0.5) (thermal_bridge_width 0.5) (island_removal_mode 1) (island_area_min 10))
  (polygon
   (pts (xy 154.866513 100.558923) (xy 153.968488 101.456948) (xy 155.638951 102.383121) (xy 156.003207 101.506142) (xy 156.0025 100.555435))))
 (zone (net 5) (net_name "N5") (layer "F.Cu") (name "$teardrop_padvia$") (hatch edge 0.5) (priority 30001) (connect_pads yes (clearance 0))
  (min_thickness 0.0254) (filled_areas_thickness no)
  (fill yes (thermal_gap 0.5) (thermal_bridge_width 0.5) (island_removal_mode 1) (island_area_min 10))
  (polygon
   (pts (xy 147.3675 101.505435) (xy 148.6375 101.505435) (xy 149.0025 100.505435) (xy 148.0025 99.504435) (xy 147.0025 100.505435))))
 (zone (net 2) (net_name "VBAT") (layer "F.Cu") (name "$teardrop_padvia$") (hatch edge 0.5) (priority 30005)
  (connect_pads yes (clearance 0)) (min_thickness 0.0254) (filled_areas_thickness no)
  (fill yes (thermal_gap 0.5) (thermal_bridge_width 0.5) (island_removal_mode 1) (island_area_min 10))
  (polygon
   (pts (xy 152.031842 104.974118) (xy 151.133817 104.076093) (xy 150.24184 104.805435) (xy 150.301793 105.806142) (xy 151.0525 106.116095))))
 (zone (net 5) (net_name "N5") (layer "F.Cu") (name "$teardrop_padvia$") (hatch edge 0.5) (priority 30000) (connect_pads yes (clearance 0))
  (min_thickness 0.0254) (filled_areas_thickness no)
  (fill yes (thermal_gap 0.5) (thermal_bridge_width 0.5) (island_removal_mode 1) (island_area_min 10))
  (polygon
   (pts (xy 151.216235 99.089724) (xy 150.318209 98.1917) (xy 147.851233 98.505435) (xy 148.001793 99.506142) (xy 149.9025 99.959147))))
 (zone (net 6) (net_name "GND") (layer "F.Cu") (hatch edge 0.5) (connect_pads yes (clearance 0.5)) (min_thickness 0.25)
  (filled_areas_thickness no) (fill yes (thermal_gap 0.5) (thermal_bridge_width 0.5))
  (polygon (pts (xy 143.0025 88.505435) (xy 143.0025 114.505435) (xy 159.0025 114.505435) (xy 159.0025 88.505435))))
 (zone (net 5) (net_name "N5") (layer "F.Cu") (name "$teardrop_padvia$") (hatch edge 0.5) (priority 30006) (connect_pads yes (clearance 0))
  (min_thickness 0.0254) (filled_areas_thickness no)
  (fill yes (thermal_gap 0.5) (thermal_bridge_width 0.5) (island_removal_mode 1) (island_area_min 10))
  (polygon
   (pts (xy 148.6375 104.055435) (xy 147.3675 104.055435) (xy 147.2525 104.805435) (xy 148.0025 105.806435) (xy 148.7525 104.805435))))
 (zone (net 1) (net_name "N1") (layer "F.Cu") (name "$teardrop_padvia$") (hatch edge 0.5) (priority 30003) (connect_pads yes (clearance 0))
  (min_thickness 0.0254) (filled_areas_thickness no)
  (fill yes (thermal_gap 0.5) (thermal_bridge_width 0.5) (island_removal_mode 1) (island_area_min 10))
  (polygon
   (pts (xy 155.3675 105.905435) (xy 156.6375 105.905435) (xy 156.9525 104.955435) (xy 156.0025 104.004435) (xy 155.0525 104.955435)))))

